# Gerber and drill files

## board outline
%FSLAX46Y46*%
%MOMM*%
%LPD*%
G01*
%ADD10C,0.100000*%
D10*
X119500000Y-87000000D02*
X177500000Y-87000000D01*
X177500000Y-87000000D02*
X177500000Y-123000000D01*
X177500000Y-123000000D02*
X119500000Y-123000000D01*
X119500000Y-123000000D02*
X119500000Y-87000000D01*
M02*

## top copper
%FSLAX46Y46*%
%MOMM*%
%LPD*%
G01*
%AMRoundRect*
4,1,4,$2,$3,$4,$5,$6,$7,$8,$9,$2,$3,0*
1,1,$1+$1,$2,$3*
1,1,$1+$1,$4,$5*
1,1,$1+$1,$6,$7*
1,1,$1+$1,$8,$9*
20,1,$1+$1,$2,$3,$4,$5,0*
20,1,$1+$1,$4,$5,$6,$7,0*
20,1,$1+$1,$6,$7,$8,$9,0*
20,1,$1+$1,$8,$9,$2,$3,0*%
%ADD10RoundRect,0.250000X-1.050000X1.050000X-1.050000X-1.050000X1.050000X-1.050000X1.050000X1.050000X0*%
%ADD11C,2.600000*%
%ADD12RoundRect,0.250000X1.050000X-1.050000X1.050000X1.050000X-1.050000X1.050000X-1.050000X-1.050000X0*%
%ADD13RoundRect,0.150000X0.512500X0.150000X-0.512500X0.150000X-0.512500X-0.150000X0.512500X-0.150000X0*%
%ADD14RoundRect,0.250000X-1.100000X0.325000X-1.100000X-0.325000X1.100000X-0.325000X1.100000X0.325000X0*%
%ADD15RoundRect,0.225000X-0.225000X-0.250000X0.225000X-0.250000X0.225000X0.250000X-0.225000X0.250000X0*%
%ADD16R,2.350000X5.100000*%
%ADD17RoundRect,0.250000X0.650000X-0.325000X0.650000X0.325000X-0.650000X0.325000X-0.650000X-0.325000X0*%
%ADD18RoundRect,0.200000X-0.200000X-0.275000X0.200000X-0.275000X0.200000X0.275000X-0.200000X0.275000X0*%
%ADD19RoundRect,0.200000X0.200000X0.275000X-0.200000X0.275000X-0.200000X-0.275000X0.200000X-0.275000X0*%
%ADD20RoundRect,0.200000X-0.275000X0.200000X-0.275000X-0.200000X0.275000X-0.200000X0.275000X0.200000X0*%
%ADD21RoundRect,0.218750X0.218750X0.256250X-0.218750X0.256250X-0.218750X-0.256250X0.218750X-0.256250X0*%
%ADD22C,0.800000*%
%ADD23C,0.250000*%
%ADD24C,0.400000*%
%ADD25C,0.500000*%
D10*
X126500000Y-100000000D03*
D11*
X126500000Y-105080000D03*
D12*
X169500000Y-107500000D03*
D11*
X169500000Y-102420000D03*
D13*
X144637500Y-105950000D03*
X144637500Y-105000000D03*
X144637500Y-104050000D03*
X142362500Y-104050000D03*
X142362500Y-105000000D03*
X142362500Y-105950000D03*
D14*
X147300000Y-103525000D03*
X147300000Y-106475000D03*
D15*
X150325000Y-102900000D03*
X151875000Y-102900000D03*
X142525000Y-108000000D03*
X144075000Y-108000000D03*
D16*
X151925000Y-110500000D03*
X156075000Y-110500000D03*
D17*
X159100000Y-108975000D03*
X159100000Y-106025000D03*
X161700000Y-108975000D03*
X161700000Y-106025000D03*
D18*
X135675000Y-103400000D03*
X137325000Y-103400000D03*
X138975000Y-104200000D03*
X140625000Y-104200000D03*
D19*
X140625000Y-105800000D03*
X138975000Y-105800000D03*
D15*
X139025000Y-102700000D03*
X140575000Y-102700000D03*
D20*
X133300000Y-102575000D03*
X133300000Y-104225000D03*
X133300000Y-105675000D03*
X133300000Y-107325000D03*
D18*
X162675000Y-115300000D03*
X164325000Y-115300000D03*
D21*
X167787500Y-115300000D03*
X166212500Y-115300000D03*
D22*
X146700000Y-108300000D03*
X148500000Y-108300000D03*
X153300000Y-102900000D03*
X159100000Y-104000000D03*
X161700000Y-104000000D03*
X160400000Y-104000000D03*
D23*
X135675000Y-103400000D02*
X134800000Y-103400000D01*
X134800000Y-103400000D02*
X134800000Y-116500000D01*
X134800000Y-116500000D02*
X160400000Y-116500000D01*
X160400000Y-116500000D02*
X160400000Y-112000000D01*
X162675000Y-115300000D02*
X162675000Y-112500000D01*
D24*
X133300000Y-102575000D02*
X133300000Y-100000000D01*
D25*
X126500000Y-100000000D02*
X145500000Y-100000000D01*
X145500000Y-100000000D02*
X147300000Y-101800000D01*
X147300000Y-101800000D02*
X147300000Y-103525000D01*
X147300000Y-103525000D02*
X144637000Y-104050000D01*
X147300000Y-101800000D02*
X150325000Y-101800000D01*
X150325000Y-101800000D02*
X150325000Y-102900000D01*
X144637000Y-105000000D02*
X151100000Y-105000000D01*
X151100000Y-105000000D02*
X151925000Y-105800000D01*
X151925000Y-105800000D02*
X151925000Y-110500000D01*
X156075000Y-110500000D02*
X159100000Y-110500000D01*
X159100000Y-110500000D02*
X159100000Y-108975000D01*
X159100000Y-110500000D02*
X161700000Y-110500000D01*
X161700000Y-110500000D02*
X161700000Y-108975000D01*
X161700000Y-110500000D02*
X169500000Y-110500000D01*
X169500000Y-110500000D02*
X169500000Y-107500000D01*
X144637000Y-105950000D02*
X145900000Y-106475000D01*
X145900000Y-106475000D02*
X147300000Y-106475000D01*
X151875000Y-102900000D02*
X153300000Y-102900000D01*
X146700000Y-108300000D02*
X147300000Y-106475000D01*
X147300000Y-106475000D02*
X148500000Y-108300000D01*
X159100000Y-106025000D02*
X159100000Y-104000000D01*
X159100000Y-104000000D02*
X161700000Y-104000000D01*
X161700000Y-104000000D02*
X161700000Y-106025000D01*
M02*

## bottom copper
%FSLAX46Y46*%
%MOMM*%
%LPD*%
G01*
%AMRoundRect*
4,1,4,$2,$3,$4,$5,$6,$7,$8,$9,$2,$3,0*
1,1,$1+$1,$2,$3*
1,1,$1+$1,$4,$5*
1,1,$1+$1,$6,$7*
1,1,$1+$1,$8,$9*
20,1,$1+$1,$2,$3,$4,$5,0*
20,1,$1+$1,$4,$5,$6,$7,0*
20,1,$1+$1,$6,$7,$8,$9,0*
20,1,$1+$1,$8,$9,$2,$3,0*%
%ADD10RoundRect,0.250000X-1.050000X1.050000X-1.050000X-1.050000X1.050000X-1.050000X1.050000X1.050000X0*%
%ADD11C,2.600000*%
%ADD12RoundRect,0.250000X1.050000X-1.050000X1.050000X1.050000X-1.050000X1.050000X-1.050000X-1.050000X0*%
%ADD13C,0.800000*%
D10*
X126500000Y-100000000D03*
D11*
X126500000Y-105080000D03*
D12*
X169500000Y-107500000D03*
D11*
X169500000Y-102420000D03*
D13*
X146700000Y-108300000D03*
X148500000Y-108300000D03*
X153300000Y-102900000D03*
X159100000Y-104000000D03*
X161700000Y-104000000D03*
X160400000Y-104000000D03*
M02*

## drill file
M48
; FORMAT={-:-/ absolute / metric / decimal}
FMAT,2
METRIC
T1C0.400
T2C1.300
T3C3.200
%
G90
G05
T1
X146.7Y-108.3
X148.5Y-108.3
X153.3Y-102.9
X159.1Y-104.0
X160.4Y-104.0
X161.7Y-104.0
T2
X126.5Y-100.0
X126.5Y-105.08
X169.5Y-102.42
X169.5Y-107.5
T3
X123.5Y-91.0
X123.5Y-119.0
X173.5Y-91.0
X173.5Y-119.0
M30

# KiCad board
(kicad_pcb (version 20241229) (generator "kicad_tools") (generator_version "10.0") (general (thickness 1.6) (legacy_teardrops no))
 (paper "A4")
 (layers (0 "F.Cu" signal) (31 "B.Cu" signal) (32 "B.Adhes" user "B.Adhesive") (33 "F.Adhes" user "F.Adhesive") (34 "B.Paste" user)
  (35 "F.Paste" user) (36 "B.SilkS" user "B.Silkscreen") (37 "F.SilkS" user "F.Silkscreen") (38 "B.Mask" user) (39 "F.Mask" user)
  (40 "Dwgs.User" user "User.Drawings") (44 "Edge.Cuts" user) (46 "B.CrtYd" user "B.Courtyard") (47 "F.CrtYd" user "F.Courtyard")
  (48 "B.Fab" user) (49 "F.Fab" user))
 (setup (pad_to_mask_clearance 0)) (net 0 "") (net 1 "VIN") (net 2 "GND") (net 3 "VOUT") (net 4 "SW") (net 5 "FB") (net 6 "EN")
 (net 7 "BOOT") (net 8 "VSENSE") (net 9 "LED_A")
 (gr_line (start 119.5 87) (end 177.5 87) (stroke (width 0.1) (type default)) (layer "Edge.Cuts"))
 (gr_line (start 177.5 87) (end 177.5 123) (stroke (width 0.1) (type default)) (layer "Edge.Cuts"))
 (gr_line (start 177.5 123) (end 119.5 123) (stroke (width 0.1) (type default)) (layer "Edge.Cuts"))
 (gr_line (start 119.5 123) (end 119.5 87) (stroke (width 0.1) (type default)) (layer "Edge.Cuts"))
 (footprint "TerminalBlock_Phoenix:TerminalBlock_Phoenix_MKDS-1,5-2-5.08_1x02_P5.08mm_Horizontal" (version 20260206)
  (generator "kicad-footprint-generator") (layer "F.Cu") (at 126.5 100 -90)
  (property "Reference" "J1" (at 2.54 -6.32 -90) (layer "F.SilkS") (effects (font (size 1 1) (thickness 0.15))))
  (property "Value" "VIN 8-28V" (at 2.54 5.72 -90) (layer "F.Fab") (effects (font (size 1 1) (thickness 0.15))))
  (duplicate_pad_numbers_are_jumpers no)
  (pad "1" thru_hole roundrect (at 0 0 -90) (size 2.6 2.6) (drill 1.3) (layers "*.Cu" "*.Mask") (remove_unused_layers no)
   (roundrect_rratio 0.096154) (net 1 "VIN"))
  (pad "2" thru_hole circle (at 5.08 0 -90) (size 2.6 2.6) (drill 1.3) (layers "*.Cu" "*.Mask") (remove_unused_layers no) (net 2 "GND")))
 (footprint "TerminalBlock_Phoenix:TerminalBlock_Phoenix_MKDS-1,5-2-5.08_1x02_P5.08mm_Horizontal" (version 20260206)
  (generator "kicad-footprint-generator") (layer "F.Cu") (at 169.5 107.5 90)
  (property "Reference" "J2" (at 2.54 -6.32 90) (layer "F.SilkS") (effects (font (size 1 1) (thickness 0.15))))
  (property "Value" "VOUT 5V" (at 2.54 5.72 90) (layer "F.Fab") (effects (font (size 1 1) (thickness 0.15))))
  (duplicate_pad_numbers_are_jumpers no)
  (pad "1" thru_hole roundrect (at 0 0 90) (size 2.6 2.6) (drill 1.3) (layers "*.Cu" "*.Mask") (remove_unused_layers no)
   (roundrect_rratio 0.096154) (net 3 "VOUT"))
  (pad "2" thru_hole circle (at 5.08 0 90) (size 2.6 2.6) (drill 1.3) (layers "*.Cu" "*.Mask") (remove_unused_layers no) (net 2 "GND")))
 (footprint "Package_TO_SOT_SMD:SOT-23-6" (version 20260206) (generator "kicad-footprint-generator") (layer "F.Cu") (at 143.5 105 180)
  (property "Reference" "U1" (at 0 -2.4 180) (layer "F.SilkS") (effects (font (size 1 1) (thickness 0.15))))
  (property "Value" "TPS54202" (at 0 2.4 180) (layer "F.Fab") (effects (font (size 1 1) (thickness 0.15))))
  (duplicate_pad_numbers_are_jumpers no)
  (pad "1" smd roundrect (at -1.1375 -0.95 180) (size 1.325 0.6) (layers "F.Cu" "F.Mask" "F.Paste") (roundrect_rratio 0.25) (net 2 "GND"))
  (pad "2" smd roundrect (at -1.1375 0 180) (size 1.325 0.6) (layers "F.Cu" "F.Mask" "F.Paste") (roundrect_rratio 0.25) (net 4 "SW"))
  (pad "3" smd roundrect (at -1.1375 0.95 180) (size 1.325 0.6) (layers "F.Cu" "F.Mask" "F.Paste") (roundrect_rratio 0.25) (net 1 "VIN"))
  (pad "4" smd roundrect (at 1.1375 0.95 180) (size 1.325 0.6) (layers "F.Cu" "F.Mask" "F.Paste") (roundrect_rratio 0.25) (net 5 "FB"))
  (pad "5" smd roundrect (at 1.1375 0 180) (size 1.325 0.6) (layers "F.Cu" "F.Mask" "F.Paste") (roundrect_rratio 0.25) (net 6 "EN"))
  (pad "6" smd roundrect (at 1.1375 -0.95 180) (size 1.325 0.6) (layers "F.Cu" "F.Mask" "F.Paste") (roundrect_rratio 0.25) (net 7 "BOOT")))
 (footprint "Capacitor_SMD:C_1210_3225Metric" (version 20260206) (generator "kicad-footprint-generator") (layer "F.Cu") (at 147.3 105 -90)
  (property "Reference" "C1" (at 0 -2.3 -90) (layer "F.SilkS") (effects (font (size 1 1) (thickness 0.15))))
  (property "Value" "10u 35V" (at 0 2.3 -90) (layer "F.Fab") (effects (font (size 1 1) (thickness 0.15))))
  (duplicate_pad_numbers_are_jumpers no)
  (pad "1" smd roundrect (at -1.475 0 -90) (size 1.15 2.7) (layers "F.Cu" "F.Mask" "F.Paste") (roundrect_rratio 0.217391) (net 1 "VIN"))
  (pad "2" smd roundrect (at 1.475 0 -90) (size 1.15 2.7) (layers "F.Cu" "F.Mask" "F.Paste") (roundrect_rratio 0.217391) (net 2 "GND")))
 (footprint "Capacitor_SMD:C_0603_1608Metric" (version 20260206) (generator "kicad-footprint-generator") (layer "F.Cu") (at 151.1 102.9)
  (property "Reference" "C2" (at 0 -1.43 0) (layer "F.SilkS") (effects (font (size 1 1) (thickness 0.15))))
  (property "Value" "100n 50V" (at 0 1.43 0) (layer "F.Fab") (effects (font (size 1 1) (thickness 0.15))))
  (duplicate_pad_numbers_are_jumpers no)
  (pad "1" smd roundrect (at -0.775 0) (size 0.9 0.95) (layers "F.Cu" "F.Mask" "F.Paste") (roundrect_rratio 0.25) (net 1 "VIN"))
  (pad "2" smd roundrect (at 0.775 0) (size 0.9 0.95) (layers "F.Cu" "F.Mask" "F.Paste") (roundrect_rratio 0.25) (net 2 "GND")))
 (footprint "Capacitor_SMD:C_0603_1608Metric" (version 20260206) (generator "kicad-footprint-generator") (layer "F.Cu") (at 143.3 108)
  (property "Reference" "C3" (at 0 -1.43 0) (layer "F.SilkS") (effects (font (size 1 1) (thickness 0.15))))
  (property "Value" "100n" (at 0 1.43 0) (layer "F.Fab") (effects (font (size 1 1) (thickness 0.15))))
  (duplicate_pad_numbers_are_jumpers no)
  (pad "1" smd roundrect (at -0.775 0) (size 0.9 0.95) (layers "F.Cu" "F.Mask" "F.Paste") (roundrect_rratio 0.25) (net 7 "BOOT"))
  (pad "2" smd roundrect (at 0.775 0) (size 0.9 0.95) (layers "F.Cu" "F.Mask" "F.Paste") (roundrect_rratio 0.25) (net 4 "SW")))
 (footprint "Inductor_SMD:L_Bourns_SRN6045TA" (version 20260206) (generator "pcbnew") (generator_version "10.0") (layer "F.Cu")
  (at 154 110.5)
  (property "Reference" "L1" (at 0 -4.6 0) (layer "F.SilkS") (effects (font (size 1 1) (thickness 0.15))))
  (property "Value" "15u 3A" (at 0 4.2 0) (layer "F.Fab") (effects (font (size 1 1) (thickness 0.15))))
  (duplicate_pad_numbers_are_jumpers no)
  (pad "1" smd rect (at -2.075 0) (size 2.35 5.1) (layers "F.Cu" "F.Mask" "F.Paste") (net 4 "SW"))
  (pad "2" smd rect (at 2.075 0) (size 2.35 5.1) (layers "F.Cu" "F.Mask" "F.Paste") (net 3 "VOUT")))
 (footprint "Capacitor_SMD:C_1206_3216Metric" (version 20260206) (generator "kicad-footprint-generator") (layer "F.Cu") (at 159.1 107.5 90)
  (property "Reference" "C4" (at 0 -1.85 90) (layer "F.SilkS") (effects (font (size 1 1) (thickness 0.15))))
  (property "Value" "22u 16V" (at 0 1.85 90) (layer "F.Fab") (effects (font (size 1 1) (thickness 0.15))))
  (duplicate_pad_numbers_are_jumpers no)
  (pad "1" smd roundrect (at -1.475 0 90) (size 1.15 1.8) (layers "F.Cu" "F.Mask" "F.Paste") (roundrect_rratio 0.217391) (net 3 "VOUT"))
  (pad "2" smd roundrect (at 1.475 0 90) (size 1.15 1.8) (layers "F.Cu" "F.Mask" "F.Paste") (roundrect_rratio 0.217391) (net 2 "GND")))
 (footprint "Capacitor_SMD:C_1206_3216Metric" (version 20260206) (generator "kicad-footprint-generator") (layer "F.Cu") (at 161.7 107.5 90)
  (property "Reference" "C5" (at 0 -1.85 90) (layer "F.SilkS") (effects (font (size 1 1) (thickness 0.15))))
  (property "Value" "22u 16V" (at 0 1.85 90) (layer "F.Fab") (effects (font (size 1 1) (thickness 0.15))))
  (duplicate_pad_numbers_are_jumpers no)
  (pad "1" smd roundrect (at -1.475 0 90) (size 1.15 1.8) (layers "F.Cu" "F.Mask" "F.Paste") (roundrect_rratio 0.217391) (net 3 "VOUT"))
  (pad "2" smd roundrect (at 1.475 0 90) (size 1.15 1.8) (layers "F.Cu" "F.Mask" "F.Paste") (roundrect_rratio 0.217391) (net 2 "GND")))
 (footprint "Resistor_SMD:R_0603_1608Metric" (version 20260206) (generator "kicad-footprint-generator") (layer "F.Cu") (at 136.5 103.4)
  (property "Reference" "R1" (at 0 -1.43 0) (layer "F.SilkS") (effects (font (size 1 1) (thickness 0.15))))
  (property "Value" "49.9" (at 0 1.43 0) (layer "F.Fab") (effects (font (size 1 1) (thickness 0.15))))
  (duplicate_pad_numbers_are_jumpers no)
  (pad "1" smd roundrect (at -0.825 0) (size 0.8 0.95) (layers "F.Cu" "F.Mask" "F.Paste") (roundrect_rratio 0.25) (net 3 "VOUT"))
  (pad "2" smd roundrect (at 0.825 0) (size 0.8 0.95) (layers "F.Cu" "F.Mask" "F.Paste") (roundrect_rratio 0.25) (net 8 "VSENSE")))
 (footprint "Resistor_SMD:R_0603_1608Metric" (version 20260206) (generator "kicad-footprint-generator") (layer "F.Cu") (at 139.8 104.2)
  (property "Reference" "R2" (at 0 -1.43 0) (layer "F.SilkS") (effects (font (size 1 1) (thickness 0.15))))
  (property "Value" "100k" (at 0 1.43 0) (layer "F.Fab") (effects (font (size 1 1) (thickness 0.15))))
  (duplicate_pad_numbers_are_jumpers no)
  (pad "1" smd roundrect (at -0.825 0) (size 0.8 0.95) (layers "F.Cu" "F.Mask" "F.Paste") (roundrect_rratio 0.25) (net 8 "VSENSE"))
  (pad "2" smd roundrect (at 0.825 0) (size 0.8 0.95) (layers "F.Cu" "F.Mask" "F.Paste") (roundrect_rratio 0.25) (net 5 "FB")))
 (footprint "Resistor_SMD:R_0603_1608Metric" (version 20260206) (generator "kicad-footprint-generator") (layer "F.Cu") (at 139.8 105.8 180)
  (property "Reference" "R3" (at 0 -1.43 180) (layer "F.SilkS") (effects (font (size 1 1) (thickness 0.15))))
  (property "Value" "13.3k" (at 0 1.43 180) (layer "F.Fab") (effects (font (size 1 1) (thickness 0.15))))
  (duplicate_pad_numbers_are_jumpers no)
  (pad "1" smd roundrect (at -0.825 0 180) (size 0.8 0.95) (layers "F.Cu" "F.Mask" "F.Paste") (roundrect_rratio 0.25) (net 5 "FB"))
  (pad "2" smd roundrect (at 0.825 0 180) (size 0.8 0.95) (layers "F.Cu" "F.Mask" "F.Paste") (roundrect_rratio 0.25) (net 2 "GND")))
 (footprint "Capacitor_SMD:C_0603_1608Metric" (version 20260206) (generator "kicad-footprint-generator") (layer "F.Cu") (at 139.8 102.7)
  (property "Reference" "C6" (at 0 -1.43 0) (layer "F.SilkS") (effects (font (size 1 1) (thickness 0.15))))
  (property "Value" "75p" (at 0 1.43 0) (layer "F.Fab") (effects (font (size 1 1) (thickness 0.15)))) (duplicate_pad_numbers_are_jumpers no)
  (pad "1" smd roundrect (at -0.775 0) (size 0.9 0.95) (layers "F.Cu" "F.Mask" "F.Paste") (roundrect_rratio 0.25) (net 8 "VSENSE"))
  (pad "2" smd roundrect (at 0.775 0) (size 0.9 0.95) (layers "F.Cu" "F.Mask" "F.Paste") (roundrect_rratio 0.25) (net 5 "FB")))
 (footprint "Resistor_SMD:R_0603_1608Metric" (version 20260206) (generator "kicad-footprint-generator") (layer "F.Cu") (at 133.3 103.4 -90)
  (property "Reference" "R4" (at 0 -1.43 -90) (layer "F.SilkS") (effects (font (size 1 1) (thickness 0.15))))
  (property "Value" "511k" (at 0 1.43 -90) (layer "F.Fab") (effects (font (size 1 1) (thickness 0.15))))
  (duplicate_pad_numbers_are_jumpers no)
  (pad "1" smd roundrect (at -0.825 0 -90) (size 0.8 0.95) (layers "F.Cu" "F.Mask" "F.Paste") (roundrect_rratio 0.25) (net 1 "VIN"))
  (pad "2" smd roundrect (at 0.825 0 -90) (size 0.8 0.95) (layers "F.Cu" "F.Mask" "F.Paste") (roundrect_rratio 0.25) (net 6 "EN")))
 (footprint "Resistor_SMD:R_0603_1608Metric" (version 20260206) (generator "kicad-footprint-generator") (layer "F.Cu") (at 133.3 106.5 -90)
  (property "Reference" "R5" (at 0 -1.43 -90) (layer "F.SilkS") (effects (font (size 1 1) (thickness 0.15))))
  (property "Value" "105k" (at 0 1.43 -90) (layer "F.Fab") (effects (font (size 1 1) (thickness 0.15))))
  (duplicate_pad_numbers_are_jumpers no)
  (pad "1" smd roundrect (at -0.825 0 -90) (size 0.8 0.95) (layers "F.Cu" "F.Mask" "F.Paste") (roundrect_rratio 0.25) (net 6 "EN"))
  (pad "2" smd roundrect (at 0.825 0 -90) (size 0.8 0.95) (layers "F.Cu" "F.Mask" "F.Paste") (roundrect_rratio 0.25) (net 2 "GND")))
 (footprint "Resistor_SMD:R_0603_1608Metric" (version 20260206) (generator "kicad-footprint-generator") (layer "F.Cu") (at 163.5 115.3)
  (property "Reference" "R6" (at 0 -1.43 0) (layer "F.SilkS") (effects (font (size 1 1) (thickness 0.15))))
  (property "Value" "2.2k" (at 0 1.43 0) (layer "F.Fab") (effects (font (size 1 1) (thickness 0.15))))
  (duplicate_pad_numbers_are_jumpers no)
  (pad "1" smd roundrect (at -0.825 0) (size 0.8 0.95) (layers "F.Cu" "F.Mask" "F.Paste") (roundrect_rratio 0.25) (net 3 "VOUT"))
  (pad "2" smd roundrect (at 0.825 0) (size 0.8 0.95) (layers "F.Cu" "F.Mask" "F.Paste") (roundrect_rratio 0.25) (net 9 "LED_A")))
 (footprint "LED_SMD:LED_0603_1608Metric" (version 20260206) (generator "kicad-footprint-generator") (layer "F.Cu") (at 167 115.3 180)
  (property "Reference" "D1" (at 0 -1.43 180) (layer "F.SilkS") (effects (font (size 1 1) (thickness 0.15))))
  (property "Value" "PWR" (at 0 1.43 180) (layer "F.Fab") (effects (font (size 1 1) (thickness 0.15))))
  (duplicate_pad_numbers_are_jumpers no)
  (pad "1" smd roundrect (at -0.7875 0 180) (size 0.875 0.95) (layers "F.Cu" "F.Mask" "F.Paste") (roundrect_rratio 0.25) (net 2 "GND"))
  (pad "2" smd roundrect (at 0.7875 0 180) (size 0.875 0.95) (layers "F.Cu" "F.Mask" "F.Paste") (roundrect_rratio 0.25) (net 9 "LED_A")))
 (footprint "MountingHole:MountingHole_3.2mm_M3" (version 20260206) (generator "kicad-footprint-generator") (layer "F.Cu") (at 123.5 91)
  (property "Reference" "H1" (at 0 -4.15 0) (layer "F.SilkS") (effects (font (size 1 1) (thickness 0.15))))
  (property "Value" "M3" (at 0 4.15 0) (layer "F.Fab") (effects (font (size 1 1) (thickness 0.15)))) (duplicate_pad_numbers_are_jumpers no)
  (pad "" np_thru_hole circle (at 0 0) (size 3.2 3.2) (drill 3.2) (layers "*.Cu" "*.Mask")))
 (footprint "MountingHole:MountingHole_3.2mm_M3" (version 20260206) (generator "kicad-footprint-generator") (layer "F.Cu") (at 173.5 91)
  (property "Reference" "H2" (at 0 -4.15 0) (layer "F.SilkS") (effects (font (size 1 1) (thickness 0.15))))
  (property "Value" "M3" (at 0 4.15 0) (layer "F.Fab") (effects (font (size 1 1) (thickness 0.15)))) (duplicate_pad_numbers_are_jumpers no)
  (pad "" np_thru_hole circle (at 0 0) (size 3.2 3.2) (drill 3.2) (layers "*.Cu" "*.Mask")))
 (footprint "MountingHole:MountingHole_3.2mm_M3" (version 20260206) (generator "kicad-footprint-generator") (layer "F.Cu") (at 123.5 119)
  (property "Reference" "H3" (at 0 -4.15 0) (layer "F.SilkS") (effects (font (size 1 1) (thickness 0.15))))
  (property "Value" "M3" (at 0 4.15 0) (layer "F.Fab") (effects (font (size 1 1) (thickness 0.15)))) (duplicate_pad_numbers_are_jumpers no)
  (pad "" np_thru_hole circle (at 0 0) (size 3.2 3.2) (drill 3.2) (layers "*.Cu" "*.Mask")))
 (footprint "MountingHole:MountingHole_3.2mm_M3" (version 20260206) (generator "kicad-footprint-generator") (layer "F.Cu") (at 173.5 119)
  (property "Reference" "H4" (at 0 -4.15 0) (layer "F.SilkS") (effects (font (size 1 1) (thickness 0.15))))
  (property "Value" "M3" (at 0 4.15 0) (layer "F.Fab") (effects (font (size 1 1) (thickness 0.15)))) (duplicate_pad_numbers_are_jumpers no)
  (pad "" np_thru_hole circle (at 0 0) (size 3.2 3.2) (drill 3.2) (layers "*.Cu" "*.Mask")))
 (via (at 146.7 108.3) (size 0.8) (drill 0.4) (layers "F.Cu" "B.Cu") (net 2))
 (via (at 148.5 108.3) (size 0.8) (drill 0.4) (layers "F.Cu" "B.Cu") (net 2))
 (via (at 153.3 102.9) (size 0.8) (drill 0.4) (layers "F.Cu" "B.Cu") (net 2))
 (via (at 159.1 104.0) (size 0.8) (drill 0.4) (layers "F.Cu" "B.Cu") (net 2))
 (via (at 161.7 104.0) (size 0.8) (drill 0.4) (layers "F.Cu" "B.Cu") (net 2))
 (via (at 160.4 104.0) (size 0.8) (drill 0.4) (layers "F.Cu" "B.Cu") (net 2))
 (segment (start 135.675 103.4) (end 134.8 103.4) (width 0.25) (layer "F.Cu") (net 3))
 (segment (start 134.8 103.4) (end 134.8 116.5) (width 0.25) (layer "F.Cu") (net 3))
 (segment (start 134.8 116.5) (end 160.4 116.5) (width 0.25) (layer "F.Cu") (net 3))
 (segment (start 160.4 116.5) (end 160.4 112.0) (width 0.25) (layer "F.Cu") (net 3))
 (segment (start 162.675 115.3) (end 162.675 112.5) (width 0.25) (layer "F.Cu") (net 3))
 (segment (start 133.3 102.575) (end 133.3 100.0) (width 0.4) (layer "F.Cu") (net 1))
 (segment (start 126.5 100.0) (end 145.5 100.0) (width 0.5) (layer "F.Cu") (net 1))
 (segment (start 145.5 100.0) (end 147.3 101.8) (width 0.5) (layer "F.Cu") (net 1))
 (segment (start 147.3 101.8) (end 147.3 103.525) (width 0.5) (layer "F.Cu") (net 1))
 (segment (start 147.3 103.525) (end 144.637 104.05) (width 0.5) (layer "F.Cu") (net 1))
 (segment (start 147.3 101.8) (end 150.325 101.8) (width 0.5) (layer "F.Cu") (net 1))
 (segment (start 150.325 101.8) (end 150.325 102.9) (width 0.5) (layer "F.Cu") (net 1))
 (segment (start 144.637 105.0) (end 151.1 105.0) (width 0.5) (layer "F.Cu") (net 4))
 (segment (start 151.1 105.0) (end 151.925 105.8) (width 0.5) (layer "F.Cu") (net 4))
 (segment (start 151.925 105.8) (end 151.925 110.5) (width 0.5) (layer "F.Cu") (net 4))
 (segment (start 156.075 110.5) (end 159.1 110.5) (width 0.5) (layer "F.Cu") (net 3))
 (segment (start 159.1 110.5) (end 159.1 108.975) (width 0.5) (layer "F.Cu") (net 3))
 (segment (start 159.1 110.5) (end 161.7 110.5) (width 0.5) (layer "F.Cu") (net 3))
 (segment (start 161.7 110.5) (end 161.7 108.975) (width 0.5) (layer "F.Cu") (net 3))
 (segment (start 161.7 110.5) (end 169.5 110.5) (width 0.5) (layer "F.Cu") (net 3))
 (segment (start 169.5 110.5) (end 169.5 107.5) (width 0.5) (layer "F.Cu") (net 3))
 (segment (start 144.637 105.95) (end 145.9 106.475) (width 0.5) (layer "F.Cu") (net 2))
 (segment (start 145.9 106.475) (end 147.3 106.475) (width 0.5) (layer "F.Cu") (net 2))
 (segment (start 151.875 102.9) (end 153.3 102.9) (width 0.5) (layer "F.Cu") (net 2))
 (segment (start 146.7 108.3) (end 147.3 106.475) (width 0.5) (layer "F.Cu") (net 2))
 (segment (start 147.3 106.475) (end 148.5 108.3) (width 0.5) (layer "F.Cu") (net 2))
 (segment (start 159.1 106.025) (end 159.1 104.0) (width 0.5) (layer "F.Cu") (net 2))
 (segment (start 159.1 104.0) (end 161.7 104.0) (width 0.5) (layer "F.Cu") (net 2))
 (segment (start 161.7 104.0) (end 161.7 106.025) (width 0.5) (layer "F.Cu") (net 2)))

